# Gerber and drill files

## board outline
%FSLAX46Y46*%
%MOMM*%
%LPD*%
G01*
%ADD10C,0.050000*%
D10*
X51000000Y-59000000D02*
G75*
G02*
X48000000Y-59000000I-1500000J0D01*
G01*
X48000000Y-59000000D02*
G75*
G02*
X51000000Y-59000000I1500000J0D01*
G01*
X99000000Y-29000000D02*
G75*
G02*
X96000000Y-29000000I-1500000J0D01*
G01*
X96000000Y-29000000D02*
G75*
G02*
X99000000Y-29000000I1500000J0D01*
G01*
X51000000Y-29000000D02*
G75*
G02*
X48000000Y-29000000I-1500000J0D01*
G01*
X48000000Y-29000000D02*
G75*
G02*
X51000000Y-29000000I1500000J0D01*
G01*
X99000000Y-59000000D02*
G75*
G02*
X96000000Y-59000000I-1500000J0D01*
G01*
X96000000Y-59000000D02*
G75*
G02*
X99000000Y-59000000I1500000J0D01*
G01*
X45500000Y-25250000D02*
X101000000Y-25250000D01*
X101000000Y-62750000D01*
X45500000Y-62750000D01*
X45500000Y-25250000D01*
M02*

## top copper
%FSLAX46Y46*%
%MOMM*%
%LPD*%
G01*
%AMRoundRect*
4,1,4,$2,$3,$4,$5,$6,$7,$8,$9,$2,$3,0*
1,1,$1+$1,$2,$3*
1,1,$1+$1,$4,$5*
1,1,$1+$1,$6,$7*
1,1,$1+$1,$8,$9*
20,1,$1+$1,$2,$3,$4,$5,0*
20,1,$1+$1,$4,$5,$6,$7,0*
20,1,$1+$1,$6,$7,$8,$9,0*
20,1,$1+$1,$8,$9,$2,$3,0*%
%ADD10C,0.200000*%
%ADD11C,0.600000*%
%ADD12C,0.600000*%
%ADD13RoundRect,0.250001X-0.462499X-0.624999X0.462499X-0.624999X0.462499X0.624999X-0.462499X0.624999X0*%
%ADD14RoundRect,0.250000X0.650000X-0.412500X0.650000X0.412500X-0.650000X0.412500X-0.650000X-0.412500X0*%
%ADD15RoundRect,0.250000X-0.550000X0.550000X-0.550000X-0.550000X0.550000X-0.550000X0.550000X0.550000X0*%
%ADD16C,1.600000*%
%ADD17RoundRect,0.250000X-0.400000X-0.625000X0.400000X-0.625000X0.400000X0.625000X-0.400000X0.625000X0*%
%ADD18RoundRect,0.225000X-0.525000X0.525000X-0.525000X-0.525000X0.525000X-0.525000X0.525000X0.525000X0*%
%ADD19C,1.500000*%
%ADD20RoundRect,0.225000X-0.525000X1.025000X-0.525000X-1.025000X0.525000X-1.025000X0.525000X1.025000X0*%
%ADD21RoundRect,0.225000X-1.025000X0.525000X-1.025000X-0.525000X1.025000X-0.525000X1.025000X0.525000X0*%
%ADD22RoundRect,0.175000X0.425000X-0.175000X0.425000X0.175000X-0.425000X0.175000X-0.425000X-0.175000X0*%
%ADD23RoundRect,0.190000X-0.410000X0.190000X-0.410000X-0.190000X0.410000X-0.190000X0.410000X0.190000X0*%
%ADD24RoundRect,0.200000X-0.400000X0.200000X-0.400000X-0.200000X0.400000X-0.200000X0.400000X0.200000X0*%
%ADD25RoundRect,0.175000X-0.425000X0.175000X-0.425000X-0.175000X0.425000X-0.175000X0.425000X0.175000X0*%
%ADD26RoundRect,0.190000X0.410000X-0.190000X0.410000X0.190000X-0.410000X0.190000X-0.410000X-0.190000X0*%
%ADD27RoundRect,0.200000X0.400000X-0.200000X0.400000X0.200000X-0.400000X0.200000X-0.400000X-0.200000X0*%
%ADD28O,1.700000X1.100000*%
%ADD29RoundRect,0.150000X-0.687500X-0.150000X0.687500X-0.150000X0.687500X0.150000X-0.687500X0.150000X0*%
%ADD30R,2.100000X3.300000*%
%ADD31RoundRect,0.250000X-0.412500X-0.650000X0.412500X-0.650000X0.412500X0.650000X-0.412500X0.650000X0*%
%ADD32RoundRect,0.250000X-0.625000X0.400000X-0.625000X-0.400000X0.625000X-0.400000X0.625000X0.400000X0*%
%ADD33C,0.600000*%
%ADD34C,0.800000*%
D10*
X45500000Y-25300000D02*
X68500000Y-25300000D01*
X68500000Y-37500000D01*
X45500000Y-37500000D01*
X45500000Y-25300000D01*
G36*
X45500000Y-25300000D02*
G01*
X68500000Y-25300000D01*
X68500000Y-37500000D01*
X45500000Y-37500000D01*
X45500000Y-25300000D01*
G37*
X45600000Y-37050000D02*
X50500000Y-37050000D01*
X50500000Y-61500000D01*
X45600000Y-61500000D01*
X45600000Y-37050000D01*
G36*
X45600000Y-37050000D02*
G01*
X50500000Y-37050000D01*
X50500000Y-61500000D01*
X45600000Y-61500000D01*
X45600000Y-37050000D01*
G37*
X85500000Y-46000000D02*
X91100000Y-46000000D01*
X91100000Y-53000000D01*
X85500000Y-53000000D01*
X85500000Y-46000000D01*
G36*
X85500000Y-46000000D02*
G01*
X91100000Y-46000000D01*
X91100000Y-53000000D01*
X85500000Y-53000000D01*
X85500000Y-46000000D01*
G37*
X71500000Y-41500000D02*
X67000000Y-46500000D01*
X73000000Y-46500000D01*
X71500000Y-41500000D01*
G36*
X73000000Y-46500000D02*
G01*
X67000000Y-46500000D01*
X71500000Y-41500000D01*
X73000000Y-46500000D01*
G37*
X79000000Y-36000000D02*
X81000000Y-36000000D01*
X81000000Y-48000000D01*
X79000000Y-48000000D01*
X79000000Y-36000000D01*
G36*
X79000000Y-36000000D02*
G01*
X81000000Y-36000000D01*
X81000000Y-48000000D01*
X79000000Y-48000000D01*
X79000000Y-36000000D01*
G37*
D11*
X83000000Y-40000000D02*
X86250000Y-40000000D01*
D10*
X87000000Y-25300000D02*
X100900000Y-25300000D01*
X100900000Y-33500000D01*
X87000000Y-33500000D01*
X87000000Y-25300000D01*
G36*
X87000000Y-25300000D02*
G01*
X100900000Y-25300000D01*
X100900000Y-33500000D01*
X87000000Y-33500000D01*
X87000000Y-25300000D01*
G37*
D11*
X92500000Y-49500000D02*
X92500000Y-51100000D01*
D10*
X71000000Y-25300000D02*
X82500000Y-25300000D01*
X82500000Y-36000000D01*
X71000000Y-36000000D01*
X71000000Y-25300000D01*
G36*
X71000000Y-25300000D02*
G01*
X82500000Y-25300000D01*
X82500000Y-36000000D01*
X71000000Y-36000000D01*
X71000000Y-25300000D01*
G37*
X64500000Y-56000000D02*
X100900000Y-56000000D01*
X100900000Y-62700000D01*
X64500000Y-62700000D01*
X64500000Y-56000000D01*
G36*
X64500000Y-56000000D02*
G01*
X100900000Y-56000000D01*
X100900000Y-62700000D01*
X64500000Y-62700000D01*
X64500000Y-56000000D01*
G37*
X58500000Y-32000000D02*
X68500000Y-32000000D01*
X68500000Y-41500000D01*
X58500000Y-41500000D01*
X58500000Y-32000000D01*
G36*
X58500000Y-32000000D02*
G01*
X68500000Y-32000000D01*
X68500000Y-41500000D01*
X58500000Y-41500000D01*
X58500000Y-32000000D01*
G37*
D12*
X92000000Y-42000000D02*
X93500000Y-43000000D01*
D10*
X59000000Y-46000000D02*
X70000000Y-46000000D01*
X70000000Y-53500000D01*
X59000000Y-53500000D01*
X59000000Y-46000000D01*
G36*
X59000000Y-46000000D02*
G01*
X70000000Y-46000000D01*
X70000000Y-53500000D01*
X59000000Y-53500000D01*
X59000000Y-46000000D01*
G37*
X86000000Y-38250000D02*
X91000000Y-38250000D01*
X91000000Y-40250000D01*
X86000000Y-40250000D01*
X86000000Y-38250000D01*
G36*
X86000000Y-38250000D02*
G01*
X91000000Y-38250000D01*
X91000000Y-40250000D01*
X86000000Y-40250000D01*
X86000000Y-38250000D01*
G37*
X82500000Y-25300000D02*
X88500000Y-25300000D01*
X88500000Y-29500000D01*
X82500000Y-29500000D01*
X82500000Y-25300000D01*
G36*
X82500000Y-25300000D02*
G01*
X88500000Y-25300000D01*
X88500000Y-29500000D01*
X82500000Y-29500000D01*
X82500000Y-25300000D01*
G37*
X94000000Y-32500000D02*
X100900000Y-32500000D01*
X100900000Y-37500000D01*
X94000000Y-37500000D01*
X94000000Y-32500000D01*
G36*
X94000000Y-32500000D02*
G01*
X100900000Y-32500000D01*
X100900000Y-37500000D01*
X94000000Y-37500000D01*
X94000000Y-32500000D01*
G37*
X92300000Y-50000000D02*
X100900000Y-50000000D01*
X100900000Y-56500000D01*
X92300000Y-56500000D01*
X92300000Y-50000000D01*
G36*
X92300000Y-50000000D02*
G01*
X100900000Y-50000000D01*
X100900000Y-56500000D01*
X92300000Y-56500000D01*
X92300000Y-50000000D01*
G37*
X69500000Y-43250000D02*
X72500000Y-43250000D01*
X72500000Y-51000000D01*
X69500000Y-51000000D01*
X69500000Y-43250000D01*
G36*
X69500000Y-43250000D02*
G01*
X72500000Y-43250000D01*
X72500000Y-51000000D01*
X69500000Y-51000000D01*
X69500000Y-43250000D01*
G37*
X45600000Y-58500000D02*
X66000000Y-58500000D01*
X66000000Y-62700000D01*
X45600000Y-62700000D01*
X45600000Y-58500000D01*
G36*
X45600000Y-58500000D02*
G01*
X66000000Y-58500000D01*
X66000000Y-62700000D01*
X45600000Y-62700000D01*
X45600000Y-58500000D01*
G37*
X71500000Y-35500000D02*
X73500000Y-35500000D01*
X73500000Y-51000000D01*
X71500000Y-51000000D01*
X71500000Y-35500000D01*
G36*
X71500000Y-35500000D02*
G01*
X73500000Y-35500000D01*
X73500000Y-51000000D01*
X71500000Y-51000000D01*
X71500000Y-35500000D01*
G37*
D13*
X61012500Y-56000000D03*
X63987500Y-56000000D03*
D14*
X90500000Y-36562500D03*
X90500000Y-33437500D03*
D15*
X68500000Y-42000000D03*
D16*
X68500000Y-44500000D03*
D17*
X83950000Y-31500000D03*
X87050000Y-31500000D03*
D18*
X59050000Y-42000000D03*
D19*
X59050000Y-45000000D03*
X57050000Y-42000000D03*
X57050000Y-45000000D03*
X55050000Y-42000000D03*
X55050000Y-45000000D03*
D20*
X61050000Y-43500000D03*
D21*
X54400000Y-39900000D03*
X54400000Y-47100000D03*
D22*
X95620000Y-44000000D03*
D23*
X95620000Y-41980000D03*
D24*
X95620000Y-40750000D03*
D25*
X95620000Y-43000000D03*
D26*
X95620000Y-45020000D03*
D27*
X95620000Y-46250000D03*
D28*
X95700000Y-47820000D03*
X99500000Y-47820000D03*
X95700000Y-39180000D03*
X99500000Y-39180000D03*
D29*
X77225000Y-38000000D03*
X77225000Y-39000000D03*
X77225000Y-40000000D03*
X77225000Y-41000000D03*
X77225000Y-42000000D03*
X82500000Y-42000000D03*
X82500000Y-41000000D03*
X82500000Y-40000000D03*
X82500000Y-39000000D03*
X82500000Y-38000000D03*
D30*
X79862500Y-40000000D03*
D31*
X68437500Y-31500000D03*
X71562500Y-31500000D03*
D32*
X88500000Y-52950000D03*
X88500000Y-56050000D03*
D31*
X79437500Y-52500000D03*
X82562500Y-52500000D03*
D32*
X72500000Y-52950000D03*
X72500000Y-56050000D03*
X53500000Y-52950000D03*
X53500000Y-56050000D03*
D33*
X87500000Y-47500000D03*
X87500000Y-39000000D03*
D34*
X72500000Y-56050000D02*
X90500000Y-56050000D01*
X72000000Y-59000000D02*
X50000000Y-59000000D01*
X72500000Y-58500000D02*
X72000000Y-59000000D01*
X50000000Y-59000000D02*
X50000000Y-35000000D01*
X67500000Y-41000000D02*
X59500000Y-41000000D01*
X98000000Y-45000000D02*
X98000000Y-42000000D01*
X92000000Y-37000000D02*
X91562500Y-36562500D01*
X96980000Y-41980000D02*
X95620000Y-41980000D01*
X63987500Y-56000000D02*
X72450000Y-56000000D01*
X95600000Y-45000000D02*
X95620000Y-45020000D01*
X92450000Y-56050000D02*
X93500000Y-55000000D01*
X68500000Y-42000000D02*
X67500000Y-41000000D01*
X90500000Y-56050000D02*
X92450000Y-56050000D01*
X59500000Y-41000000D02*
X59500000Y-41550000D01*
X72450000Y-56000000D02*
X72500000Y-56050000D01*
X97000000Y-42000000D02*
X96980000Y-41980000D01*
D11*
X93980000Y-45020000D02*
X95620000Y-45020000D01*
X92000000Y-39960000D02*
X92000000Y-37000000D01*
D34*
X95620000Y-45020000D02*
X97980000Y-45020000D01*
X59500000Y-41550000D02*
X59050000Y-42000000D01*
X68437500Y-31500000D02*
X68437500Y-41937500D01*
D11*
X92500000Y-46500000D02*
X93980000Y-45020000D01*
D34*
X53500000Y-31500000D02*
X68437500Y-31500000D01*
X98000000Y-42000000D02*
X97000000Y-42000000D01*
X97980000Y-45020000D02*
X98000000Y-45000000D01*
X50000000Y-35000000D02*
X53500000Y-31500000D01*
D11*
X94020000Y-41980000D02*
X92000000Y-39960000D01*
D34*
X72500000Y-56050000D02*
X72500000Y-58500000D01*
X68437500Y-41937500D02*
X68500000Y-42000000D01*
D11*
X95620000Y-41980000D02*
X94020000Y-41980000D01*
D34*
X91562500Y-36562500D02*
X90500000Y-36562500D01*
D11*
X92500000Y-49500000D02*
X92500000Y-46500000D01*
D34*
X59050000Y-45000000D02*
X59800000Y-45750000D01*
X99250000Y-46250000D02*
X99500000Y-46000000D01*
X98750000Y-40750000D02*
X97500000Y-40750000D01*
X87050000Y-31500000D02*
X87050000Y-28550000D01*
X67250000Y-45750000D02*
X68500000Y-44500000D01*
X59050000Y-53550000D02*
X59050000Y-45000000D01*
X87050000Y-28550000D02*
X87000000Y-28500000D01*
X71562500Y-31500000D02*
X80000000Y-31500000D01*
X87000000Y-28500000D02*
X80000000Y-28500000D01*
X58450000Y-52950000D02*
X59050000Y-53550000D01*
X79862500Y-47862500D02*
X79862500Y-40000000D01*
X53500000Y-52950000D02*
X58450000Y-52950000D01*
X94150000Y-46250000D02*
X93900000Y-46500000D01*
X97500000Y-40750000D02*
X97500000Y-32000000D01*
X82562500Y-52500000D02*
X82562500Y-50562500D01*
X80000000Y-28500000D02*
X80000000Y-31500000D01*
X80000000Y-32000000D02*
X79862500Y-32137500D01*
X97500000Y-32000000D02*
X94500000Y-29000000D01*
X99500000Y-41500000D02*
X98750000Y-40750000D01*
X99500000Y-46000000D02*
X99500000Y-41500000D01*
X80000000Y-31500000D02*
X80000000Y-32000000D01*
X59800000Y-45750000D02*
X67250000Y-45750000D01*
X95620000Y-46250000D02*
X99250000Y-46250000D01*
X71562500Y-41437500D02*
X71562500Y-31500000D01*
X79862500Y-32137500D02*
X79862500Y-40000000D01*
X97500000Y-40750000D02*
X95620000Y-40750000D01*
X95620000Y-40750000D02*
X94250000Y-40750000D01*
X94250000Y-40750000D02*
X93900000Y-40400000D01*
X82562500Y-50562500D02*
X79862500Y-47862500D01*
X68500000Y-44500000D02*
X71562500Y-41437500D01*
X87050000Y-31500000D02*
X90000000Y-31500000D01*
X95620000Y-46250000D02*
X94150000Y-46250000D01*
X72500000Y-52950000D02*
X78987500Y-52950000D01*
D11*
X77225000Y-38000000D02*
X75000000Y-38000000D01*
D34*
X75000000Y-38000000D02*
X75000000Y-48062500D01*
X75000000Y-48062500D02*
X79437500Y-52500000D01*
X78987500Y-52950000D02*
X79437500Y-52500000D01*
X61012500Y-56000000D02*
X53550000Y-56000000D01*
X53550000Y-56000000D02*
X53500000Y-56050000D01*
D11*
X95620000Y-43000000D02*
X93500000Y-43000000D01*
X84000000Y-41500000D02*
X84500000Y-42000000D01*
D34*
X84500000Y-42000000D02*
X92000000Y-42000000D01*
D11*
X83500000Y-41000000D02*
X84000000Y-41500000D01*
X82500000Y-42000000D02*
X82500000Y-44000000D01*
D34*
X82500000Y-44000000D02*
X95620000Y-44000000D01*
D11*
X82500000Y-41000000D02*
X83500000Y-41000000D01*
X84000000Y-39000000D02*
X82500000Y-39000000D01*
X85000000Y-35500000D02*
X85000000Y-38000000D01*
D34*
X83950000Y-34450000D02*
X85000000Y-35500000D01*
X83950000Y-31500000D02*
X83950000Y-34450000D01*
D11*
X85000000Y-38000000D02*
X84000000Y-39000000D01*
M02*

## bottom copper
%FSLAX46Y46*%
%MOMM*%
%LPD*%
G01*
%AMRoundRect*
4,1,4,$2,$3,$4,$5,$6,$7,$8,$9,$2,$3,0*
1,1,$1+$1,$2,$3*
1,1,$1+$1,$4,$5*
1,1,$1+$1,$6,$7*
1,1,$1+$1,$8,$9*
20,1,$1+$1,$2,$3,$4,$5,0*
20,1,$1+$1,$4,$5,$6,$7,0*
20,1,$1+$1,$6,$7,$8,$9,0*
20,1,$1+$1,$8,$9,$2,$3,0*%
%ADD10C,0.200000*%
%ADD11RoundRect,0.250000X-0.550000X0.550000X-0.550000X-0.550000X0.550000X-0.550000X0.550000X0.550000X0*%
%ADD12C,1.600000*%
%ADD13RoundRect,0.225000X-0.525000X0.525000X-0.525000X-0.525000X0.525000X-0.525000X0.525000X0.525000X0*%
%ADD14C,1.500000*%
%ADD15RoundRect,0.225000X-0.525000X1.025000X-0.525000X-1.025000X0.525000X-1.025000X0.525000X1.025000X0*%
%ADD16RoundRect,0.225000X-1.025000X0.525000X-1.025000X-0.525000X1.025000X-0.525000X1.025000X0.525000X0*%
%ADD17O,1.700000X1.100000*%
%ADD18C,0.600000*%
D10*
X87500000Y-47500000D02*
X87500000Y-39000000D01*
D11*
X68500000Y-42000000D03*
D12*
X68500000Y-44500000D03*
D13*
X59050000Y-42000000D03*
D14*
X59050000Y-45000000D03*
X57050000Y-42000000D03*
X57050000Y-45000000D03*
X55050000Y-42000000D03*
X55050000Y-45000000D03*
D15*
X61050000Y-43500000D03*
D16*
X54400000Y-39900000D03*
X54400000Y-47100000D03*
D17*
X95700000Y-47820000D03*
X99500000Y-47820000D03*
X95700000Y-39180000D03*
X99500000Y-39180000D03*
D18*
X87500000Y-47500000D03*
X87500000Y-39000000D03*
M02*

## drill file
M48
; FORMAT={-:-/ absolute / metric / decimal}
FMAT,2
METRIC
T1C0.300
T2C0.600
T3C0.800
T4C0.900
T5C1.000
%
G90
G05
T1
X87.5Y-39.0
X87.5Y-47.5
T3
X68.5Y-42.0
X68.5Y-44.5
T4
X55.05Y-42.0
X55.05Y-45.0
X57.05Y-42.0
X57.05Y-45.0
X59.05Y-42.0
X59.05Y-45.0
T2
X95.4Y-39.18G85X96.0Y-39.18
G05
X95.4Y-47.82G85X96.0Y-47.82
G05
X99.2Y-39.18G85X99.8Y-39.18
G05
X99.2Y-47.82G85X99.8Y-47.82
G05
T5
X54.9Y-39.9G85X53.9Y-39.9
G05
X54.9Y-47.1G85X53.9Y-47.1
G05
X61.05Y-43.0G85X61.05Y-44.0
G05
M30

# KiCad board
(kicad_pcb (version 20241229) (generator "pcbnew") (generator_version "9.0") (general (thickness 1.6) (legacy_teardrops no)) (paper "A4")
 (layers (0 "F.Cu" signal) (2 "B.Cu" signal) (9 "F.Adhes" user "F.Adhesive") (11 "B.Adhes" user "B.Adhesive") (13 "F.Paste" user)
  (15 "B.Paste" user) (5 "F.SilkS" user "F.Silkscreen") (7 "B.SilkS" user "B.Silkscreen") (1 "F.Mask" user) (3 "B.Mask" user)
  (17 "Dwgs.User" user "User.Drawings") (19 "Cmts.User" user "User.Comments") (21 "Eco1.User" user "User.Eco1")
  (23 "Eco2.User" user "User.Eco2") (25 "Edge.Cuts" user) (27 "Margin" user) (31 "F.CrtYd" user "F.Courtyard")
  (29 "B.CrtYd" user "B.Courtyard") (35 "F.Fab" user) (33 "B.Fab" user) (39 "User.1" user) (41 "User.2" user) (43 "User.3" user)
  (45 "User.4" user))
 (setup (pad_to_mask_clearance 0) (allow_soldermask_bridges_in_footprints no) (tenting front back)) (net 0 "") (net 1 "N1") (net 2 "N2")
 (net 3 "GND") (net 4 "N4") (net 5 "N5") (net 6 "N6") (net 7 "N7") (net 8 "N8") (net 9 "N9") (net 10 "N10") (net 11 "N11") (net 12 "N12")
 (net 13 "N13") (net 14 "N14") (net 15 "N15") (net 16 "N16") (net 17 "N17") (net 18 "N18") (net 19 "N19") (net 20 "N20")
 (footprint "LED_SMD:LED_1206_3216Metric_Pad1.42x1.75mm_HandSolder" (layer "F.Cu") (at 62.5 56)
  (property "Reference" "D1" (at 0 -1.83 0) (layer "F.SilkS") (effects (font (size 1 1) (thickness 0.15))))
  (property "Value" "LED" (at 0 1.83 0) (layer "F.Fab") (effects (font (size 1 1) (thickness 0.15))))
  (pad "1" smd roundrect (at -1.4875 0) (size 1.425 1.75) (layers "F.Cu" "F.Mask" "F.Paste") (roundrect_rratio 0.175439) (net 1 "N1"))
  (pad "2" smd roundrect (at 1.4875 0) (size 1.425 1.75) (layers "F.Cu" "F.Mask" "F.Paste") (roundrect_rratio 0.175439) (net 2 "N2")))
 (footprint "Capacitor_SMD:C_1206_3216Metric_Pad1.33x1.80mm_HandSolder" (layer "F.Cu") (at 90.5 35 90)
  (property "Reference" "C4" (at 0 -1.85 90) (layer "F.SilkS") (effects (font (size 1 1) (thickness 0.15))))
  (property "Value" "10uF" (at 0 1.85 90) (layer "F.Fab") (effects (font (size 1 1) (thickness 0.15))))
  (pad "1" smd roundrect (at -1.5625 0 90) (size 1.325 1.8) (layers "F.Cu" "F.Mask" "F.Paste") (roundrect_rratio 0.188679) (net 2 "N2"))
  (pad "2" smd roundrect (at 1.5625 0 90) (size 1.325 1.8) (layers "F.Cu" "F.Mask" "F.Paste") (roundrect_rratio 0.188679) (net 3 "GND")))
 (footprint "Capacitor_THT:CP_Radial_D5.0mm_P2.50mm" (layer "F.Cu") (at 68.5 42 -90)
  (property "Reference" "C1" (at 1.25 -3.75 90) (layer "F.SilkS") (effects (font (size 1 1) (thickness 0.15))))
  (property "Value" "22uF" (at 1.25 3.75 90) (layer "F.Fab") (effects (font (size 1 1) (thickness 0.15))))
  (pad "1" thru_hole roundrect (at 0 0 270) (size 1.6 1.6) (drill 0.8) (layers "*.Cu" "*.Mask") (remove_unused_layers no)
   (roundrect_rratio 0.15625) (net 2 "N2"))
  (pad "2" thru_hole circle (at 2.5 0 270) (size 1.6 1.6) (drill 0.8) (layers "*.Cu" "*.Mask") (remove_unused_layers no) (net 3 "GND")))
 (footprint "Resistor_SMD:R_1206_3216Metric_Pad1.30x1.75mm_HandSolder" (layer "F.Cu") (at 85.5 31.5)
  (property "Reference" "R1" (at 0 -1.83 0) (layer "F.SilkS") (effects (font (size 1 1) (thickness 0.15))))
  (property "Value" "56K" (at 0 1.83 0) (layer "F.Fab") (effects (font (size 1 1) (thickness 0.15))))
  (pad "1" smd roundrect (at -1.55 0) (size 1.3 1.75) (layers "F.Cu" "F.Mask" "F.Paste") (roundrect_rratio 0.192308) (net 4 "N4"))
  (pad "2" smd roundrect (at 1.55 0) (size 1.3 1.75) (layers "F.Cu" "F.Mask" "F.Paste") (roundrect_rratio 0.192308) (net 3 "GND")))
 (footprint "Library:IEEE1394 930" (layer "F.Cu") (at 45.5 43.5 -90)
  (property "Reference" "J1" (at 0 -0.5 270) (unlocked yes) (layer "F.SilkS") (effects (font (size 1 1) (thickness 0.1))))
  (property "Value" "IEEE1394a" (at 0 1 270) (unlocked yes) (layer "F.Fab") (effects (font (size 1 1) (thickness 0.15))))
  (pad "1" thru_hole roundrect (at -1.5 -13.55 270) (size 1.5 1.5) (drill 0.9) (layers "*.Cu" "*.Mask") (remove_unused_layers no)
   (roundrect_rratio 0.15) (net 2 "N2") (thermal_bridge_angle 45))
  (pad "2" thru_hole circle (at 1.5 -13.55 270) (size 1.5 1.5) (drill 0.9) (layers "*.Cu" "*.Mask") (remove_unused_layers no) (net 3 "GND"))
  (pad "3" thru_hole circle (at -1.5 -11.55 270) (size 1.5 1.5) (drill 0.9) (layers "*.Cu" "*.Mask") (remove_unused_layers no) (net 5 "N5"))
  (pad "4" thru_hole circle (at 1.5 -11.55 270) (size 1.5 1.5) (drill 0.9) (layers "*.Cu" "*.Mask") (remove_unused_layers no) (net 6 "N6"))
  (pad "5" thru_hole circle (at -1.5 -9.55 270) (size 1.5 1.5) (drill 0.9) (layers "*.Cu" "*.Mask") (remove_unused_layers no) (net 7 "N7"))
  (pad "6" thru_hole circle (at 1.5 -9.55 270) (size 1.5 1.5) (drill 0.9) (layers "*.Cu" "*.Mask") (remove_unused_layers no) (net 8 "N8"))
  (pad "7" thru_hole roundrect (at 0 -15.55 270) (size 2.5 1.5) (drill oval 2 1) (layers "*.Cu" "*.Mask") (remove_unused_layers no)
   (roundrect_rratio 0.15) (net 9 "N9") (thermal_bridge_angle 45))
  (pad "8" thru_hole roundrect (at -3.6 -8.9 270) (size 1.5 2.5) (drill oval 1 2) (layers "*.Cu" "*.Mask") (remove_unused_layers no)
   (roundrect_rratio 0.15) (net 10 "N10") (thermal_bridge_angle 45))
  (pad "9" thru_hole roundrect (at 3.6 -8.9 270) (size 1.5 2.5) (drill oval 1 2) (layers "*.Cu" "*.Mask") (remove_unused_layers no)
   (roundrect_rratio 0.15) (thermal_bridge_angle 45)))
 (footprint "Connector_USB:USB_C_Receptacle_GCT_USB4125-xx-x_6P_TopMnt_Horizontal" (layer "F.Cu") (at 98.7 43.5 90)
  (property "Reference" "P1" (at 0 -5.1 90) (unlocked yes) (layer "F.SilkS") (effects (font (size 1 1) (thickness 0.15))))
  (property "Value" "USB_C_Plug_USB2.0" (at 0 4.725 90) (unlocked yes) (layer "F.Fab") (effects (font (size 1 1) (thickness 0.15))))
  (pad "A5" smd roundrect (at -0.5 -3.08 90) (size 0.7 1.2) (layers "F.Cu" "F.Mask" "F.Paste") (roundrect_rratio 0.25) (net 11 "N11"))
  (pad "A9" smd roundrect (at 1.52 -3.08 270) (size 0.76 1.2) (layers "F.Cu" "F.Mask" "F.Paste") (roundrect_rratio 0.25) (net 2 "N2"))
  (pad "A12" smd roundrect (at 2.75 -3.08 270) (size 0.8 1.2) (layers "F.Cu" "F.Mask" "F.Paste") (roundrect_rratio 0.25) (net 3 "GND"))
  (pad "B5" smd roundrect (at 0.5 -3.08 270) (size 0.7 1.2) (layers "F.Cu" "F.Mask" "F.Paste") (roundrect_rratio 0.25) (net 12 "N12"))
  (pad "B9" smd roundrect (at -1.52 -3.08 90) (size 0.76 1.2) (layers "F.Cu" "F.Mask" "F.Paste") (roundrect_rratio 0.25) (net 2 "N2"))
  (pad "B12" smd roundrect (at -2.75 -3.08 90) (size 0.8 1.2) (layers "F.Cu" "F.Mask" "F.Paste") (roundrect_rratio 0.25) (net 3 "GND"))
  (pad "S1" thru_hole oval (at -4.32 -3 90) (size 1.1 1.7) (drill oval 0.6 1.2) (layers "*.Cu" "*.Mask" "F.Paste") (remove_unused_layers no)
   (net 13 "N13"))
  (pad "S1" thru_hole oval (at -4.32 0.8 90) (size 1.1 1.7) (drill oval 0.6 1.2) (layers "*.Cu" "*.Mask" "F.Paste")
   (remove_unused_layers no) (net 13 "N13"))
  (pad "S1" thru_hole oval (at 4.32 -3 90) (size 1.1 1.7) (drill oval 0.6 1.2) (layers "*.Cu" "*.Mask" "F.Paste") (remove_unused_layers no)
   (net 13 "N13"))
  (pad "S1" thru_hole oval (at 4.32 0.8 90) (size 1.1 1.7) (drill oval 0.6 1.2) (layers "*.Cu" "*.Mask" "F.Paste") (remove_unused_layers no)
   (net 13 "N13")))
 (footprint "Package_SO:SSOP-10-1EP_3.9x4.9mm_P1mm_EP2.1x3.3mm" (layer "F.Cu") (at 79.8625 40)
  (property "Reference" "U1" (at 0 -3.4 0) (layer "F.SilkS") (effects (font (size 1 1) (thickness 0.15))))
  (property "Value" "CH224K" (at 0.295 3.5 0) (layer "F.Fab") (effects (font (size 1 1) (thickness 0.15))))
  (pad "" smd roundrect (at 0 0) (size 1.69 2.66) (layers "F.Paste") (roundrect_rratio 0.147929))
  (pad "1" smd roundrect (at -2.6375 -2) (size 1.675 0.6) (layers "F.Cu" "F.Mask" "F.Paste") (roundrect_rratio 0.25) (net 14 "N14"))
  (pad "2" smd roundrect (at -2.6375 -1) (size 1.675 0.6) (layers "F.Cu" "F.Mask" "F.Paste") (roundrect_rratio 0.25) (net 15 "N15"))
  (pad "3" smd roundrect (at -2.6375 0) (size 1.675 0.6) (layers "F.Cu" "F.Mask" "F.Paste") (roundrect_rratio 0.25) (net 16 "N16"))
  (pad "4" smd roundrect (at -2.6375 1) (size 1.675 0.6) (layers "F.Cu" "F.Mask" "F.Paste") (roundrect_rratio 0.25) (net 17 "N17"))
  (pad "5" smd roundrect (at -2.6375 2) (size 1.675 0.6) (layers "F.Cu" "F.Mask" "F.Paste") (roundrect_rratio 0.25) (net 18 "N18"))
  (pad "6" smd roundrect (at 2.6375 2) (size 1.675 0.6) (layers "F.Cu" "F.Mask" "F.Paste") (roundrect_rratio 0.25) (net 11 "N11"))
  (pad "7" smd roundrect (at 2.6375 1) (size 1.675 0.6) (layers "F.Cu" "F.Mask" "F.Paste") (roundrect_rratio 0.25) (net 11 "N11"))
  (pad "8" smd roundrect (at 2.6375 0) (size 1.675 0.6) (layers "F.Cu" "F.Mask" "F.Paste") (roundrect_rratio 0.25) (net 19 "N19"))
  (pad "9" smd roundrect (at 2.6375 -1) (size 1.675 0.6) (layers "F.Cu" "F.Mask" "F.Paste") (roundrect_rratio 0.25) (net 4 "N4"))
  (pad "10" smd roundrect (at 2.6375 -2) (size 1.675 0.6) (layers "F.Cu" "F.Mask" "F.Paste") (roundrect_rratio 0.25) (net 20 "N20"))
  (pad "11" smd rect (at 0 0) (size 2.1 3.3) (layers "F.Cu" "F.Mask") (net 3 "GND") (zone_connect 2)))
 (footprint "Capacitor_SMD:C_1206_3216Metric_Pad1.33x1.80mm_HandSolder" (layer "F.Cu") (at 70 31.5)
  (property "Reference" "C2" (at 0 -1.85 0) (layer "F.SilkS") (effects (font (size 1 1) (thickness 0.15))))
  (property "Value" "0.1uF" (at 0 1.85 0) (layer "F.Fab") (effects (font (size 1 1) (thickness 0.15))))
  (pad "1" smd roundrect (at -1.5625 0) (size 1.325 1.8) (layers "F.Cu" "F.Mask" "F.Paste") (roundrect_rratio 0.188679) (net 2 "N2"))
  (pad "2" smd roundrect (at 1.5625 0) (size 1.325 1.8) (layers "F.Cu" "F.Mask" "F.Paste") (roundrect_rratio 0.188679) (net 3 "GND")))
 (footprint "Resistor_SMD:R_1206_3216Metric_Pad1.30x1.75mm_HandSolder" (layer "F.Cu") (at 88.5 54.5 -90)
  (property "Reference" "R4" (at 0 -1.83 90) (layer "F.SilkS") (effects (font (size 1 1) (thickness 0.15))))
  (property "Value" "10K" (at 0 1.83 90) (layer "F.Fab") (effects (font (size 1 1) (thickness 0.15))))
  (pad "1" smd roundrect (at -1.55 0 270) (size 1.3 1.75) (layers "F.Cu" "F.Mask" "F.Paste") (roundrect_rratio 0.192308) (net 19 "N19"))
  (pad "2" smd roundrect (at 1.55 0 270) (size 1.3 1.75) (layers "F.Cu" "F.Mask" "F.Paste") (roundrect_rratio 0.192308) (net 2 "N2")))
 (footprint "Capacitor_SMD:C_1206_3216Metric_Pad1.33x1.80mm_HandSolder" (layer "F.Cu") (at 81 52.5)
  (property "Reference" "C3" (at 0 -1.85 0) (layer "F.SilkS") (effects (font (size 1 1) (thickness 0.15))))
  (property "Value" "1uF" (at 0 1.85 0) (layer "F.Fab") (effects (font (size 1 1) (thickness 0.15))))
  (pad "1" smd roundrect (at -1.5625 0) (size 1.325 1.8) (layers "F.Cu" "F.Mask" "F.Paste") (roundrect_rratio 0.188679) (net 14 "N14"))
  (pad "2" smd roundrect (at 1.5625 0) (size 1.325 1.8) (layers "F.Cu" "F.Mask" "F.Paste") (roundrect_rratio 0.188679) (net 3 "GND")))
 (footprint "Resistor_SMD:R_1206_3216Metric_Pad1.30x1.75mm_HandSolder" (layer "F.Cu") (at 72.5 54.5 -90)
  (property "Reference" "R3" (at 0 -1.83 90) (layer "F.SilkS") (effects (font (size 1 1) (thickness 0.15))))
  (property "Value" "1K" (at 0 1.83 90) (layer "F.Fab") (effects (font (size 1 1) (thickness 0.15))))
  (pad "1" smd roundrect (at -1.55 0 270) (size 1.3 1.75) (layers "F.Cu" "F.Mask" "F.Paste") (roundrect_rratio 0.192308) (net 14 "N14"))
  (pad "2" smd roundrect (at 1.55 0 270) (size 1.3 1.75) (layers "F.Cu" "F.Mask" "F.Paste") (roundrect_rratio 0.192308) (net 2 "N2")))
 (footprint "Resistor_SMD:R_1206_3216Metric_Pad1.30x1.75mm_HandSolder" (layer "F.Cu") (at 53.5 54.5 -90)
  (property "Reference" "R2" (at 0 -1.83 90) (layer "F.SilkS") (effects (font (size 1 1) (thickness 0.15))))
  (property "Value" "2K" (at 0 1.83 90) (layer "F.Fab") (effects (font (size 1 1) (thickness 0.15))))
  (pad "1" smd roundrect (at -1.55 0 270) (size 1.3 1.75) (layers "F.Cu" "F.Mask" "F.Paste") (roundrect_rratio 0.192308) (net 3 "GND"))
  (pad "2" smd roundrect (at 1.55 0 270) (size 1.3 1.75) (layers "F.Cu" "F.Mask" "F.Paste") (roundrect_rratio 0.192308) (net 1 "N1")))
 (gr_rect (start 45.5 25.3) (end 68.5 37.5) (stroke (width 0.2) (type solid)) (fill yes) (layer "F.Cu") (net 2))
 (gr_rect (start 45.6 37.05) (end 50.5 61.5) (stroke (width 0.2) (type solid)) (fill yes) (layer "F.Cu") (net 2))
 (gr_rect (start 85.5 46) (end 91.1 53) (stroke (width 0.2) (type solid)) (fill yes) (layer "F.Cu") (net 19))
 (gr_poly (pts (xy 71.5 41.5) (xy 67 46.5) (xy 73 46.5)) (stroke (width 0.2) (type solid)) (fill yes) (layer "F.Cu") (net 3))
 (gr_rect (start 79 36) (end 81 48) (stroke (width 0.2) (type solid)) (fill yes) (layer "F.Cu") (net 3))
 (gr_line (start 83 40) (end 86.25 40) (stroke (width 0.6) (type solid)) (layer "F.Cu") (net 19))
 (gr_rect (start 87 25.3) (end 100.9 33.5) (stroke (width 0.2) (type solid)) (fill yes) (layer "F.Cu") (net 3))
 (gr_line (start 92.5 49.5) (end 92.5 51.1) (stroke (width 0.6) (type solid)) (layer "F.Cu") (net 2))
 (gr_rect (start 71 25.3) (end 82.5 36) (stroke (width 0.2) (type solid)) (fill yes) (layer "F.Cu") (net 3))
 (gr_rect (start 64.5 56) (end 100.9 62.7) (stroke (width 0.2) (type solid)) (fill yes) (layer "F.Cu") (net 2))
 (gr_rect (start 58.5 32) (end 68.5 41.5) (stroke (width 0.2) (type solid)) (fill yes) (layer "F.Cu") (net 2))
 (gr_line (start 92 42) (end 93.5 43) (stroke (width 0.6) (type solid)) (layer "F.Cu"))
 (gr_rect (start 59 46) (end 70 53.5) (stroke (width 0.2) (type solid)) (fill yes) (layer "F.Cu") (net 3))
 (gr_rect (start 86 38.25) (end 91 40.25) (stroke (width 0.2) (type solid)) (fill yes) (layer "F.Cu") (net 19))
 (gr_rect (start 82.5 25.3) (end 88.5 29.5) (stroke (width 0.2) (type solid)) (fill yes) (layer "F.Cu") (net 3))
 (gr_rect (start 94 32.5) (end 100.9 37.5) (stroke (width 0.2) (type solid)) (fill yes) (layer "F.Cu") (net 3))
 (gr_rect (start 92.3 50) (end 100.9 56.5) (stroke (width 0.2) (type solid)) (fill yes) (layer "F.Cu") (net 2))
 (gr_rect (start 69.5 43.25) (end 72.5 51) (stroke (width 0.2) (type solid)) (fill yes) (layer "F.Cu") (net 3))
 (gr_rect (start 45.6 58.5) (end 66 62.7) (stroke (width 0.2) (type solid)) (fill yes) (layer "F.Cu") (net 2))
 (gr_rect (start 71.5 35.5) (end 73.5 51) (stroke (width 0.2) (type solid)) (fill yes) (layer "F.Cu") (net 3))
 (gr_line (start 87.5 47.5) (end 87.5 39) (stroke (width 0.2) (type default)) (layer "B.Cu") (net 19))
 (gr_circle (center 49.5 59) (end 48 59) (stroke (width 0.05) (type default)) (fill no) (layer "Edge.Cuts"))
 (gr_circle (center 97.5 29) (end 99 29) (stroke (width 0.05) (type default)) (fill no) (layer "Edge.Cuts"))
 (gr_circle (center 49.5 29) (end 51 29) (stroke (width 0.05) (type solid)) (fill no) (layer "Edge.Cuts"))
 (gr_circle (center 97.5 59) (end 99 59) (stroke (width 0.05) (type default)) (fill no) (layer "Edge.Cuts"))
 (gr_rect (start 45.5 25.25) (end 101 62.75) (stroke (width 0.05) (type default)) (fill no) (layer "Edge.Cuts"))
 (segment (start 72.5 56.05) (end 90.5 56.05) (width 0.8) (layer "F.Cu") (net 2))
 (segment (start 72 59) (end 50 59) (width 0.8) (layer "F.Cu") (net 2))
 (segment (start 72.5 58.5) (end 72 59) (width 0.8) (layer "F.Cu") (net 2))
 (segment (start 50 59) (end 50 35) (width 0.8) (layer "F.Cu") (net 2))
 (segment (start 67.5 41) (end 59.5 41) (width 0.8) (layer "F.Cu") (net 2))
 (segment (start 98 45) (end 98 42) (width 0.8) (layer "F.Cu") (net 2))
 (segment (start 92 37) (end 91.5625 36.5625) (width 0.8) (layer "F.Cu") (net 2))
 (segment (start 96.98 41.98) (end 95.62 41.98) (width 0.8) (layer "F.Cu") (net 2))
 (segment (start 63.9875 56) (end 72.45 56) (width 0.8) (layer "F.Cu") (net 2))
 (segment (start 95.6 45) (end 95.62 45.02) (width 0.8) (layer "F.Cu") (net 2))
 (segment (start 92.45 56.05) (end 93.5 55) (width 0.8) (layer "F.Cu") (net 2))
 (segment (start 68.5 42) (end 67.5 41) (width 0.8) (layer "F.Cu") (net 2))
 (segment (start 90.5 56.05) (end 92.45 56.05) (width 0.8) (layer "F.Cu") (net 2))
 (segment (start 59.5 41) (end 59.5 41.55) (width 0.8) (layer "F.Cu") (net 2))
 (segment (start 72.45 56) (end 72.5 56.05) (width 0.8) (layer "F.Cu") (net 2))
 (segment (start 97 42) (end 96.98 41.98) (width 0.8) (layer "F.Cu") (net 2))
 (segment (start 93.98 45.02) (end 95.62 45.02) (width 0.6) (layer "F.Cu") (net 2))
 (segment (start 92 39.96) (end 92 37) (width 0.6) (layer "F.Cu") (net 2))
 (segment (start 95.62 45.02) (end 97.98 45.02) (width 0.8) (layer "F.Cu") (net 2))
 (segment (start 59.5 41.55) (end 59.05 42) (width 0.8) (layer "F.Cu") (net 2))
 (segment (start 68.4375 31.5) (end 68.4375 41.9375) (width 0.8) (layer "F.Cu") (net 2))
 (segment (start 92.5 46.5) (end 93.98 45.02) (width 0.6) (layer "F.Cu") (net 2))
 (segment (start 53.5 31.5) (end 68.4375 31.5) (width 0.8) (layer "F.Cu") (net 2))
 (segment (start 98 42) (end 97 42) (width 0.8) (layer "F.Cu") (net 2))
 (segment (start 97.98 45.02) (end 98 45) (width 0.8) (layer "F.Cu") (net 2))
 (segment (start 50 35) (end 53.5 31.5) (width 0.8) (layer "F.Cu") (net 2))
 (segment (start 94.02 41.98) (end 92 39.96) (width 0.6) (layer "F.Cu") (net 2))
 (segment (start 72.5 56.05) (end 72.5 58.5) (width 0.8) (layer "F.Cu") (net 2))
 (segment (start 68.4375 41.9375) (end 68.5 42) (width 0.8) (layer "F.Cu") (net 2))
 (segment (start 95.62 41.98) (end 94.02 41.98) (width 0.6) (layer "F.Cu") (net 2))
 (segment (start 91.5625 36.5625) (end 90.5 36.5625) (width 0.8) (layer "F.Cu") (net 2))
 (segment (start 92.5 49.5) (end 92.5 46.5) (width 0.6) (layer "F.Cu") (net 2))
 (segment (start 59.05 45) (end 59.8 45.75) (width 0.8) (layer "F.Cu") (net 3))
 (segment (start 99.25 46.25) (end 99.5 46) (width 0.8) (layer "F.Cu") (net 3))
 (segment (start 98.75 40.75) (end 97.5 40.75) (width 0.8) (layer "F.Cu") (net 3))
 (segment (start 87.05 31.5) (end 87.05 28.55) (width 0.8) (layer "F.Cu") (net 3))
 (segment (start 67.25 45.75) (end 68.5 44.5) (width 0.8) (layer "F.Cu") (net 3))
 (segment (start 59.05 53.55) (end 59.05 45) (width 0.8) (layer "F.Cu") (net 3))
 (segment (start 87.05 28.55) (end 87 28.5) (width 0.8) (layer "F.Cu") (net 3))
 (segment (start 71.5625 31.5) (end 80 31.5) (width 0.8) (layer "F.Cu") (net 3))
 (segment (start 87 28.5) (end 80 28.5) (width 0.8) (layer "F.Cu") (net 3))
 (segment (start 58.45 52.95) (end 59.05 53.55) (width 0.8) (layer "F.Cu") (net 3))
 (segment (start 79.8625 47.8625) (end 79.8625 40) (width 0.8) (layer "F.Cu") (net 3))
 (segment (start 53.5 52.95) (end 58.45 52.95) (width 0.8) (layer "F.Cu") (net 3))
 (segment (start 94.15 46.25) (end 93.9 46.5) (width 0.8) (layer "F.Cu") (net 3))
 (segment (start 97.5 40.75) (end 97.5 32) (width 0.8) (layer "F.Cu") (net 3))
 (segment (start 82.5625 52.5) (end 82.5625 50.5625) (width 0.8) (layer "F.Cu") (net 3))
 (segment (start 80 28.5) (end 80 31.5) (width 0.8) (layer "F.Cu") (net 3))
 (segment (start 80 32) (end 79.8625 32.1375) (width 0.8) (layer "F.Cu") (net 3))
 (segment (start 97.5 32) (end 94.5 29) (width 0.8) (layer "F.Cu") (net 3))
 (segment (start 99.5 41.5) (end 98.75 40.75) (width 0.8) (layer "F.Cu") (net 3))
 (segment (start 99.5 46) (end 99.5 41.5) (width 0.8) (layer "F.Cu") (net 3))
 (segment (start 80 31.5) (end 80 32) (width 0.8) (layer "F.Cu") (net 3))
 (segment (start 59.8 45.75) (end 67.25 45.75) (width 0.8) (layer "F.Cu") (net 3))
 (segment (start 95.62 46.25) (end 99.25 46.25) (width 0.8) (layer "F.Cu") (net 3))
 (segment (start 71.5625 41.4375) (end 71.5625 31.5) (width 0.8) (layer "F.Cu") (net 3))
 (segment (start 79.8625 32.1375) (end 79.8625 40) (width 0.8) (layer "F.Cu") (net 3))
 (segment (start 97.5 40.75) (end 95.62 40.75) (width 0.8) (layer "F.Cu") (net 3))
 (segment (start 95.62 40.75) (end 94.25 40.75) (width 0.8) (layer "F.Cu") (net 3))
 (segment (start 94.25 40.75) (end 93.9 40.4) (width 0.8) (layer "F.Cu") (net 3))
 (segment (start 82.5625 50.5625) (end 79.8625 47.8625) (width 0.8) (layer "F.Cu") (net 3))
 (segment (start 68.5 44.5) (end 71.5625 41.4375) (width 0.8) (layer "F.Cu") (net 3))
 (segment (start 87.05 31.5) (end 90 31.5) (width 0.8) (layer "F.Cu") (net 3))
 (segment (start 95.62 46.25) (end 94.15 46.25) (width 0.8) (layer "F.Cu") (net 3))
 (segment (start 72.5 52.95) (end 78.9875 52.95) (width 0.8) (layer "F.Cu") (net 14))
 (segment (start 77.225 38) (end 75 38) (width 0.6) (layer "F.Cu") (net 14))
 (segment (start 75 38) (end 75 48.0625) (width 0.8) (layer "F.Cu") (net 14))
 (segment (start 75 48.0625) (end 79.4375 52.5) (width 0.8) (layer "F.Cu") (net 14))
 (segment (start 78.9875 52.95) (end 79.4375 52.5) (width 0.8) (layer "F.Cu") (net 14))
 (segment (start 61.0125 56) (end 53.55 56) (width 0.8) (layer "F.Cu") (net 1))
 (segment (start 53.55 56) (end 53.5 56.05) (width 0.8) (layer "F.Cu") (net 1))
 (segment (start 95.62 43) (end 93.5 43) (width 0.6) (layer "F.Cu") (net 12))
 (segment (start 84 41.5) (end 84.5 42) (width 0.6) (layer "F.Cu") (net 11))
 (segment (start 84.5 42) (end 92 42) (width 0.8) (layer "F.Cu") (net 11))
 (segment (start 83.5 41) (end 84 41.5) (width 0.6) (layer "F.Cu") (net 11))
 (segment (start 82.5 42) (end 82.5 44) (width 0.6) (layer "F.Cu") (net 11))
 (segment (start 82.5 44) (end 95.62 44) (width 0.8) (layer "F.Cu") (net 11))
 (segment (start 82.5 41) (end 83.5 41) (width 0.6) (layer "F.Cu") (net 11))
 (segment (start 84 39) (end 82.5 39) (width 0.6) (layer "F.Cu") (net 4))
 (segment (start 85 35.5) (end 85 38) (width 0.6) (layer "F.Cu") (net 4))
 (segment (start 83.95 34.45) (end 85 35.5) (width 0.8) (layer "F.Cu") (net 4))
 (segment (start 83.95 31.5) (end 83.95 34.45) (width 0.8) (layer "F.Cu") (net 4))
 (segment (start 85 38) (end 84 39) (width 0.6) (layer "F.Cu") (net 4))
 (via (at 87.5 47.5) (size 0.6) (drill 0.3) (layers "F.Cu" "B.Cu") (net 19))
 (via (at 87.5 39) (size 0.6) (drill 0.3) (layers "F.Cu" "B.Cu") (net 19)))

